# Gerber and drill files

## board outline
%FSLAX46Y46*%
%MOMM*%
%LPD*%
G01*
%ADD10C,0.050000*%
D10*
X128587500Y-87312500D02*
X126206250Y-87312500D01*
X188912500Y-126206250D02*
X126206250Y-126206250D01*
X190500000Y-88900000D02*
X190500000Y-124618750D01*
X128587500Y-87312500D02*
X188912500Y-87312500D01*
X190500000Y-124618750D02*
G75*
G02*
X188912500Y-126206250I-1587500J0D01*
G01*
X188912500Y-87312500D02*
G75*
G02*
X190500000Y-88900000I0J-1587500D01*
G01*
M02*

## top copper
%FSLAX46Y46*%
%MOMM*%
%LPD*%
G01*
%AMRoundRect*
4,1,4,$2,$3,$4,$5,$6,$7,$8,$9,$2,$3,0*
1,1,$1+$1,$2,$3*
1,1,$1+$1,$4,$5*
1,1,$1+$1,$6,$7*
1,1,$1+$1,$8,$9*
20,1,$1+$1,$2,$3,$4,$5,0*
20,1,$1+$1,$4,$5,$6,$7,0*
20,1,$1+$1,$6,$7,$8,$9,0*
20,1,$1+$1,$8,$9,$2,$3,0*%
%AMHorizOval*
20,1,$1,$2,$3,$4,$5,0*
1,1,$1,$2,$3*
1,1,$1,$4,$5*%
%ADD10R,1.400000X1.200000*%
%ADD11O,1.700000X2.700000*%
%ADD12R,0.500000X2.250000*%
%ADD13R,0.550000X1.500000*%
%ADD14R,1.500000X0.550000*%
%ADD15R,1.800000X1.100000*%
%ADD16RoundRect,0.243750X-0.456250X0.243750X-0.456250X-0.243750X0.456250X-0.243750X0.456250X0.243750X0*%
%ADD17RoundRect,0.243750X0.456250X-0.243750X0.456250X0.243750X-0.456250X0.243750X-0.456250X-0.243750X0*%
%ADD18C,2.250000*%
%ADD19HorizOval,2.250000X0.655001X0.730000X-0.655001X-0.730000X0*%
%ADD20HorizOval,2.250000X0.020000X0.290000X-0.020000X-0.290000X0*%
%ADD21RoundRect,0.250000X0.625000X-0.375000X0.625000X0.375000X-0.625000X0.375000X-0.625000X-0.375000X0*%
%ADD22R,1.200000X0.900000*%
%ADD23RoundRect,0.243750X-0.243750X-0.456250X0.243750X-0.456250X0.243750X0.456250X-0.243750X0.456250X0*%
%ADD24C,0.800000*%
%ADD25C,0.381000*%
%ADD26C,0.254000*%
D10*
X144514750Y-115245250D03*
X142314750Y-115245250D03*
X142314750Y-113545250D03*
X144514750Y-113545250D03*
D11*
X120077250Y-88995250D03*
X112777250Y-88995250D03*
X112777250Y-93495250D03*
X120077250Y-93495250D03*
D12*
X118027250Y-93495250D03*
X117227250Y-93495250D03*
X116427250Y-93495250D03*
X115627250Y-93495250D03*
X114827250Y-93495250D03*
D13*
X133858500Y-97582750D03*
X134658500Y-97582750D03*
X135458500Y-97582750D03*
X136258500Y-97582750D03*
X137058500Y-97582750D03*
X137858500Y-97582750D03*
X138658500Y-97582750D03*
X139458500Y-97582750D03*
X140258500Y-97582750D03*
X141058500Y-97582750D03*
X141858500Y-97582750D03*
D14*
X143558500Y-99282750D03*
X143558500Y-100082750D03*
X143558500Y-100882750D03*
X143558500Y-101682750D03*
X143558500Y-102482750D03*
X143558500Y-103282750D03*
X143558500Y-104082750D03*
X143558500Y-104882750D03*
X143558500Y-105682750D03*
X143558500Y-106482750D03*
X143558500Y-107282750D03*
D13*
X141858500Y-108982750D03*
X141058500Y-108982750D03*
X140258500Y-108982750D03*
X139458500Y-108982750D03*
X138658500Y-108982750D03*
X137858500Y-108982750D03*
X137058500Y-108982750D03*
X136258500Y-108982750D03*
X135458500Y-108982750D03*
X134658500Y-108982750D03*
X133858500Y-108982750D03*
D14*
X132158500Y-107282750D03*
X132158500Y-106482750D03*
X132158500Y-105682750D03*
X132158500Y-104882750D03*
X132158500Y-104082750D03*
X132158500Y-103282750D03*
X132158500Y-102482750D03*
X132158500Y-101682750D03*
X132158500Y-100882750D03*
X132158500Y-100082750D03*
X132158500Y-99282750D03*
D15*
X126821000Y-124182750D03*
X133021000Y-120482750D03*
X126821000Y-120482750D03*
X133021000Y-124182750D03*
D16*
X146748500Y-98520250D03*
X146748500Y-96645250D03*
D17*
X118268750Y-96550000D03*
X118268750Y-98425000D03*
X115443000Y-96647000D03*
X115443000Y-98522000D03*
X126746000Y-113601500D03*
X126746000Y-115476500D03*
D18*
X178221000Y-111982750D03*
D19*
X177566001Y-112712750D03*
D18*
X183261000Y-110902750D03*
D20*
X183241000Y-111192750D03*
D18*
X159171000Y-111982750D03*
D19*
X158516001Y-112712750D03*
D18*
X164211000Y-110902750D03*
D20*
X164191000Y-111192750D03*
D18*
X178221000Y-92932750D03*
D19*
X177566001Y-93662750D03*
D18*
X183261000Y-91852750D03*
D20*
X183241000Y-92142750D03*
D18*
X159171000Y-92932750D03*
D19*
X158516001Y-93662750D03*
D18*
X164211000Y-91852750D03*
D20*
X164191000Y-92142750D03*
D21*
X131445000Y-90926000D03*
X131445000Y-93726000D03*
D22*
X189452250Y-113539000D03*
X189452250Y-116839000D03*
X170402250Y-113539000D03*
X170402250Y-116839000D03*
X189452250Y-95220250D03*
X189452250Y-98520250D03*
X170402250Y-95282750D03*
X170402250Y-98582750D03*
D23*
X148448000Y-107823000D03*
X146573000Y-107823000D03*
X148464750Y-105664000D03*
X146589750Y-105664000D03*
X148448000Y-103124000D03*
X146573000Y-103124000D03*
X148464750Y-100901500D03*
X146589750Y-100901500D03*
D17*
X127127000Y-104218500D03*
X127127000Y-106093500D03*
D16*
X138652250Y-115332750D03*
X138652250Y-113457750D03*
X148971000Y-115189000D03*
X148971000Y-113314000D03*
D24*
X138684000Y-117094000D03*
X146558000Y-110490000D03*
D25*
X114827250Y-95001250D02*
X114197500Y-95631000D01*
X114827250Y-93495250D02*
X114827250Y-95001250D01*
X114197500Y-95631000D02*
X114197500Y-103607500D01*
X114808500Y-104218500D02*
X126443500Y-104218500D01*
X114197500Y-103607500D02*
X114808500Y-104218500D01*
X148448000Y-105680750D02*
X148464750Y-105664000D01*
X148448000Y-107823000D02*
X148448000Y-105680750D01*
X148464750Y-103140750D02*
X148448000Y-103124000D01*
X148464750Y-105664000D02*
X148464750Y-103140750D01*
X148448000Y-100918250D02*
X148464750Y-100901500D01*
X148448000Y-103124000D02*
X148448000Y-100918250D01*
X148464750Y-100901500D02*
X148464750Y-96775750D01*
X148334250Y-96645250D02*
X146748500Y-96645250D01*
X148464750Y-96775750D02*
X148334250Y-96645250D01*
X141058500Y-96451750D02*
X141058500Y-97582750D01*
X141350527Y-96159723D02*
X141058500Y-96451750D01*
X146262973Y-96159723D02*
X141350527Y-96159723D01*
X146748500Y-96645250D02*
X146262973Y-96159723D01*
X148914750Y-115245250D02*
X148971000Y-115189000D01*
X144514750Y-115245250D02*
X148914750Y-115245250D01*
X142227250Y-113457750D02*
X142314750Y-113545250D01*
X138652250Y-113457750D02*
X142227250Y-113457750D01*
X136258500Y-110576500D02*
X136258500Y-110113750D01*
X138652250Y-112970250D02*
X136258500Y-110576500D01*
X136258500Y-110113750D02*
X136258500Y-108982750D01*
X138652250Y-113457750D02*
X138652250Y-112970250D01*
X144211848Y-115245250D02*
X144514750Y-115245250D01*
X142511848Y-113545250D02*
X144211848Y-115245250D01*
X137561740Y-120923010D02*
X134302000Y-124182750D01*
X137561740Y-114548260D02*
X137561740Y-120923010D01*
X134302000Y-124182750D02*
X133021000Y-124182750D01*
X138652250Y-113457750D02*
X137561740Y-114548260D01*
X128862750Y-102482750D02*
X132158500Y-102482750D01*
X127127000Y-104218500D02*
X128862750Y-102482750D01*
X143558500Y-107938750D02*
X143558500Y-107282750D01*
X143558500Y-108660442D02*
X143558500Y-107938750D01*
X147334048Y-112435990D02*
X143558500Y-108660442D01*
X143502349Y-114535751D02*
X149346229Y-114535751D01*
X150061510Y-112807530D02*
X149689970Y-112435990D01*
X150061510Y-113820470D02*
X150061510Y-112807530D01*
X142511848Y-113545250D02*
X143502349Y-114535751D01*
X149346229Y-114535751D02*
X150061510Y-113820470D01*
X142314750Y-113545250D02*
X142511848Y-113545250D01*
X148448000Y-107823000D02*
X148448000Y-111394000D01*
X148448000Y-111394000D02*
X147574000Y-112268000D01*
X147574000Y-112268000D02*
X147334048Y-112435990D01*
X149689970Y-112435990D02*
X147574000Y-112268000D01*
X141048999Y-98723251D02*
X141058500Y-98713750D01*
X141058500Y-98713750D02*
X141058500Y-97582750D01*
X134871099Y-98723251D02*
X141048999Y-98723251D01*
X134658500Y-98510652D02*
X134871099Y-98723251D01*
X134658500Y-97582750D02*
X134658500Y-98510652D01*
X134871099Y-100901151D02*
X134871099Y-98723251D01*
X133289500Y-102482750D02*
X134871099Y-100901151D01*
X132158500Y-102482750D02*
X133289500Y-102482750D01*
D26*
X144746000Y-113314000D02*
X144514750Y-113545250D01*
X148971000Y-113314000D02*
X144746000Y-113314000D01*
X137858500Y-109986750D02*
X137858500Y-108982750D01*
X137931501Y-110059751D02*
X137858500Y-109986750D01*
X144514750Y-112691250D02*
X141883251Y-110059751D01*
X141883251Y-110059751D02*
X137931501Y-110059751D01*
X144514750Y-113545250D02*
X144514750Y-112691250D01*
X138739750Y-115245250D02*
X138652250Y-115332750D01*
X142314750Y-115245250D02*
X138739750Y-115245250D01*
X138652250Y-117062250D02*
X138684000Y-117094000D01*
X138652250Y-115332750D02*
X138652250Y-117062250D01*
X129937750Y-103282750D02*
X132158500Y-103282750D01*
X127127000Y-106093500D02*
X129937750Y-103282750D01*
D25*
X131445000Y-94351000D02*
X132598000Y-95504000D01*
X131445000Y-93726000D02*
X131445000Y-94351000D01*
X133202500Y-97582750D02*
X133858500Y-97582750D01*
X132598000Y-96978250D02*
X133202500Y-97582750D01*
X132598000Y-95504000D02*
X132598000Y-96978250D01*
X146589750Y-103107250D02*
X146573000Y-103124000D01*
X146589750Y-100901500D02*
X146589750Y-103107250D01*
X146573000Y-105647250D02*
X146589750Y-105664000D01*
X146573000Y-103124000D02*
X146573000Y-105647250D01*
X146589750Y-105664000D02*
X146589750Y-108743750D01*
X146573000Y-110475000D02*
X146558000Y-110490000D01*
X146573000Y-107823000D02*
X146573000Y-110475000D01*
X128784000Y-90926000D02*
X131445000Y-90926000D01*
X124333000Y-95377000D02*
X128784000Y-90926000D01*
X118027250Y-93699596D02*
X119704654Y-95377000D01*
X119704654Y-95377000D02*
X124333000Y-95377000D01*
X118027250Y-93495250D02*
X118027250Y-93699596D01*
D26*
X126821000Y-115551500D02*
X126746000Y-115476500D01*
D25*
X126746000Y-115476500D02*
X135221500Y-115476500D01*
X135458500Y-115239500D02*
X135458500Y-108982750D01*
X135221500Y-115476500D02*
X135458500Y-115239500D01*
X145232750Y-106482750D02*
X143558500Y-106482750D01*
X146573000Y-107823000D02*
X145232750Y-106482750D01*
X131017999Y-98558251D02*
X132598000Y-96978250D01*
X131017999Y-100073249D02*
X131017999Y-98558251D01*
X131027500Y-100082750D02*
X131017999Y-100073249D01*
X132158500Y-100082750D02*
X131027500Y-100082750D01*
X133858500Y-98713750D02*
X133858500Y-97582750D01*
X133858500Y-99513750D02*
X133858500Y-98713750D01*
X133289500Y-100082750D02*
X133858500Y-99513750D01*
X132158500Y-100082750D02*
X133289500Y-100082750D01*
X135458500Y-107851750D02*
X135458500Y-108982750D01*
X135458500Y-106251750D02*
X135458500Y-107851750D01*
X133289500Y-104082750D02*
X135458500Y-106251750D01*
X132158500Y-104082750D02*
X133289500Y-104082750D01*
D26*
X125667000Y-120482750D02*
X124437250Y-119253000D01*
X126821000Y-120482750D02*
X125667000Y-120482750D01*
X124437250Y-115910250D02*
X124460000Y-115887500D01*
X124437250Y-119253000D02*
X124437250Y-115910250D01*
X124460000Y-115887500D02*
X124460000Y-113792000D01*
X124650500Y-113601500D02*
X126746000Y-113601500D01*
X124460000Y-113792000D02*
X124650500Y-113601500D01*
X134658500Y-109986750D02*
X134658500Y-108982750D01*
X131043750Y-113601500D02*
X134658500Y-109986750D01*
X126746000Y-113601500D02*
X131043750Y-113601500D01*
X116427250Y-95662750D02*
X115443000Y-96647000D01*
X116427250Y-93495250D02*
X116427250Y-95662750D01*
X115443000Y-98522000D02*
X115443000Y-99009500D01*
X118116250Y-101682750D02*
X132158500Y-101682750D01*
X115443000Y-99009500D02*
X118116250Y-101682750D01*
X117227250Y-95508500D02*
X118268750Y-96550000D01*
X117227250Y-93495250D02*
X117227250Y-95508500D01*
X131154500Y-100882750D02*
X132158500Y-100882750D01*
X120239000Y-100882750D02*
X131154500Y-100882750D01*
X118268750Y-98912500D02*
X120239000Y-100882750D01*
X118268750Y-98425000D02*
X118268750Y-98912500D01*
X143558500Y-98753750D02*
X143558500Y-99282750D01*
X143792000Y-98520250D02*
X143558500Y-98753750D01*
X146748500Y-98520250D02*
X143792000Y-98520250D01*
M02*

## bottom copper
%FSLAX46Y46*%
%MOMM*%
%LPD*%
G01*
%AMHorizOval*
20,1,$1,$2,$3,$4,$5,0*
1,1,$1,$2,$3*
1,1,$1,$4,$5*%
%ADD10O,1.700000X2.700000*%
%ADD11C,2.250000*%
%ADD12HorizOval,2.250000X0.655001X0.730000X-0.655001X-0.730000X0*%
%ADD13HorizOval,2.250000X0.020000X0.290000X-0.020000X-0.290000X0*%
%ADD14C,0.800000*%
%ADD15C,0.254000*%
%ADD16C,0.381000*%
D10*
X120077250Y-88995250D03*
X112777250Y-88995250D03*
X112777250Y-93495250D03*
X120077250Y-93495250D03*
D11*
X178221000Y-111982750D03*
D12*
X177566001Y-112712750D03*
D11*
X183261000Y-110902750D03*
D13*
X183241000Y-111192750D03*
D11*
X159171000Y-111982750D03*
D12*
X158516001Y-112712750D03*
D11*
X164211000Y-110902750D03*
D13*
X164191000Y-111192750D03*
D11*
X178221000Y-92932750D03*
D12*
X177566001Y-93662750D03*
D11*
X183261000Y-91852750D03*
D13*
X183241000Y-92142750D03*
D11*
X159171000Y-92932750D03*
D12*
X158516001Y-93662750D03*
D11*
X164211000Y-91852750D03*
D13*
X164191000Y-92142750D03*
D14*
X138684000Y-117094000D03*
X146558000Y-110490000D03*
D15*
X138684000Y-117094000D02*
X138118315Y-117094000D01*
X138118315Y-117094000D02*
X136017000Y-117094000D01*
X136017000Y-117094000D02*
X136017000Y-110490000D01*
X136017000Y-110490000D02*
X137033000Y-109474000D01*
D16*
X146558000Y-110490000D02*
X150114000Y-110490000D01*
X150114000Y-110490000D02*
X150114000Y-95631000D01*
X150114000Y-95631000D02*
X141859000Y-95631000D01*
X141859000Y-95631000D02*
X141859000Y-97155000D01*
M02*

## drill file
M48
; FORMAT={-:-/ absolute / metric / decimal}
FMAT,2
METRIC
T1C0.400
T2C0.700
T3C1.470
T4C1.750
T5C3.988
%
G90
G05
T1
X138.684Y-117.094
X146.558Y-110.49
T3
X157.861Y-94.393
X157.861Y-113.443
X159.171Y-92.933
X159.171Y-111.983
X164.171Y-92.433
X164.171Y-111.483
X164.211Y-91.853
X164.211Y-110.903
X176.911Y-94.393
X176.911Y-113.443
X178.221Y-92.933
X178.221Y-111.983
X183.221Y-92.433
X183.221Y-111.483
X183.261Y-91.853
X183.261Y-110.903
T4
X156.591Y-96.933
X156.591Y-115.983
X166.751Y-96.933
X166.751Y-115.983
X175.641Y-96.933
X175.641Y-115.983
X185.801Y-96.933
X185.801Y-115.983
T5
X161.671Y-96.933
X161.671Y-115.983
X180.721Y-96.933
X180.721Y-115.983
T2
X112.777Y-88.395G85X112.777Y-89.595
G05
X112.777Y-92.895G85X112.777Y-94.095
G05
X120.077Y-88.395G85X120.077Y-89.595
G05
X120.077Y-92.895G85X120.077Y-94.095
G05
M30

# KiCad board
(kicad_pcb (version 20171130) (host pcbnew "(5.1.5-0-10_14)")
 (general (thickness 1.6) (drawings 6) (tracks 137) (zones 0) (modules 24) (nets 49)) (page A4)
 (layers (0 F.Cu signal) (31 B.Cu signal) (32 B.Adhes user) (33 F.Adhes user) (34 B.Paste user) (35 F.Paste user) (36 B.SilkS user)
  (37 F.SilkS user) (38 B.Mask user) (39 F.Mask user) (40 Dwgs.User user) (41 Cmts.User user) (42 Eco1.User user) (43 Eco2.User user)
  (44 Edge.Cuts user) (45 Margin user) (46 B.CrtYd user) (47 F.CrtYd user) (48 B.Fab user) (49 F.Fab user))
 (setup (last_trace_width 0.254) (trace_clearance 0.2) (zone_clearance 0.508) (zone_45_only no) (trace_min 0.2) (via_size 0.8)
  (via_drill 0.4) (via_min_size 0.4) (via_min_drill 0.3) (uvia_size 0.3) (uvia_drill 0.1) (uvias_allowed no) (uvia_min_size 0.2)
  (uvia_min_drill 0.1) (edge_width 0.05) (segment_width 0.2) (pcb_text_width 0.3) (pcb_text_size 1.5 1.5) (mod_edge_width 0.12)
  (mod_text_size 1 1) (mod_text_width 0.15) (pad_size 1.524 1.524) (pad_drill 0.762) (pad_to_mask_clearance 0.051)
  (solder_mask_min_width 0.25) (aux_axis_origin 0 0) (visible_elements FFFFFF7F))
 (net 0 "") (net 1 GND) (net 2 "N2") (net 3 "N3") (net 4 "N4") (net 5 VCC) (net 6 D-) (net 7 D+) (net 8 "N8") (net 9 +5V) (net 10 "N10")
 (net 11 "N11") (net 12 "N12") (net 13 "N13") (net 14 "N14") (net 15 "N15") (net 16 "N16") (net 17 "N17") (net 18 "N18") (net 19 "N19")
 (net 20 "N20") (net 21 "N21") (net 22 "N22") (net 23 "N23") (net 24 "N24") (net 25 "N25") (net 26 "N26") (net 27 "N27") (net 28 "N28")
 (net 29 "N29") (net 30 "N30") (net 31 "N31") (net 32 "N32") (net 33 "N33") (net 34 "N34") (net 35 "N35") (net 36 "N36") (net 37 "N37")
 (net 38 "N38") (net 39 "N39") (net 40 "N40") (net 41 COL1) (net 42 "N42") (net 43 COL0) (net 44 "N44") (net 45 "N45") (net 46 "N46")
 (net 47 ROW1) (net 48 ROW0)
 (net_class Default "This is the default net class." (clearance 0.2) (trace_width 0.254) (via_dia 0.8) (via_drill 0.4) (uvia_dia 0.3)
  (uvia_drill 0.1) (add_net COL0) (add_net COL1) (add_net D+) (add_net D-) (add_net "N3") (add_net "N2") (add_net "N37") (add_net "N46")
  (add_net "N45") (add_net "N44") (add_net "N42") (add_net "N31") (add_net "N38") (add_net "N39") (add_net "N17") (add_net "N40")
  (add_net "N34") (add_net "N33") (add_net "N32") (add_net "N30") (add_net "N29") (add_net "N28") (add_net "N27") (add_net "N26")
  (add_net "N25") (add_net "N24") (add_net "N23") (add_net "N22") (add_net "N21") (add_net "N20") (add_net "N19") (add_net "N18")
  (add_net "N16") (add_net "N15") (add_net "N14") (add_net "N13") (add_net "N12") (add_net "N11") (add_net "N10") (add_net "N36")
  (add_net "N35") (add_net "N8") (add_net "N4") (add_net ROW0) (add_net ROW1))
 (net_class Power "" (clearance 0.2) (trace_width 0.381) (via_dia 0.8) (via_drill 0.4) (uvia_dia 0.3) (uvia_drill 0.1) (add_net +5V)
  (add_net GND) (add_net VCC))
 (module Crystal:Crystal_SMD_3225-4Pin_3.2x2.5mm (layer F.Cu) (at 143.41475 114.39525 180)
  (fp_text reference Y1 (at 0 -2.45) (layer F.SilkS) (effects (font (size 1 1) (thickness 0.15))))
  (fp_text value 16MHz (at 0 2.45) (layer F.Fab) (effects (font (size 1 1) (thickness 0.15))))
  (pad 4 smd rect (at -1.1 -0.85 180) (size 1.4 1.2) (layers F.Cu F.Paste F.Mask) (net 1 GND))
  (pad 3 smd rect (at 1.1 -0.85 180) (size 1.4 1.2) (layers F.Cu F.Paste F.Mask) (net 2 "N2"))
  (pad 2 smd rect (at 1.1 0.85 180) (size 1.4 1.2) (layers F.Cu F.Paste F.Mask) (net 1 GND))
  (pad 1 smd rect (at -1.1 0.85 180) (size 1.4 1.2) (layers F.Cu F.Paste F.Mask) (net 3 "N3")))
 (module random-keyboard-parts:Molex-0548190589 (layer F.Cu) (at 116.42725 88.99525 270)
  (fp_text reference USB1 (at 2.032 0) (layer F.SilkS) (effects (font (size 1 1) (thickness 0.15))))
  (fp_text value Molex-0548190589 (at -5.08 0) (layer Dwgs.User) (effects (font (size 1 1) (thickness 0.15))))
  (pad 6 thru_hole oval (at 0 -3.65 270) (size 2.7 1.7) (drill oval 1.9 0.7) (layers *.Cu *.Mask) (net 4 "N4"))
  (pad 6 thru_hole oval (at 0 3.65 270) (size 2.7 1.7) (drill oval 1.9 0.7) (layers *.Cu *.Mask) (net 4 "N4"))
  (pad 6 thru_hole oval (at 4.5 3.65 270) (size 2.7 1.7) (drill oval 1.9 0.7) (layers *.Cu *.Mask) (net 4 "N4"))
  (pad 6 thru_hole oval (at 4.5 -3.65 270) (size 2.7 1.7) (drill oval 1.9 0.7) (layers *.Cu *.Mask) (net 4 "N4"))
  (pad 5 smd rect (at 4.5 -1.6 270) (size 2.25 0.5) (layers F.Cu F.Paste F.Mask) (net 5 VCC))
  (pad 4 smd rect (at 4.5 -0.8 270) (size 2.25 0.5) (layers F.Cu F.Paste F.Mask) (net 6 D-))
  (pad 3 smd rect (at 4.5 0 270) (size 2.25 0.5) (layers F.Cu F.Paste F.Mask) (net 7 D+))
  (pad 2 smd rect (at 4.5 0.8 270) (size 2.25 0.5) (layers F.Cu F.Paste F.Mask) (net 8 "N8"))
  (pad 1 smd rect (at 4.5 1.6 270) (size 2.25 0.5) (layers F.Cu F.Paste F.Mask) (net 1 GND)))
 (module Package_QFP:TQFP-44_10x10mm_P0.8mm (layer F.Cu) (at 137.8585 103.28275)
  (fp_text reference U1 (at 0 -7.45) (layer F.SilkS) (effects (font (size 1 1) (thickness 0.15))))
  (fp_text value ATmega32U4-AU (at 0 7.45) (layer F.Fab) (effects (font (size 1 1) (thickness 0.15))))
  (pad 44 smd rect (at -4 -5.7 90) (size 1.5 0.55) (layers F.Cu F.Paste F.Mask) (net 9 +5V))
  (pad 43 smd rect (at -3.2 -5.7 90) (size 1.5 0.55) (layers F.Cu F.Paste F.Mask) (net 1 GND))
  (pad 42 smd rect (at -2.4 -5.7 90) (size 1.5 0.55) (layers F.Cu F.Paste F.Mask) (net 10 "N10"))
  (pad 41 smd rect (at -1.6 -5.7 90) (size 1.5 0.55) (layers F.Cu F.Paste F.Mask) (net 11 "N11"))
  (pad 40 smd rect (at -0.8 -5.7 90) (size 1.5 0.55) (layers F.Cu F.Paste F.Mask) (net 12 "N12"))
  (pad 39 smd rect (at 0 -5.7 90) (size 1.5 0.55) (layers F.Cu F.Paste F.Mask) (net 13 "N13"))
  (pad 38 smd rect (at 0.8 -5.7 90) (size 1.5 0.55) (layers F.Cu F.Paste F.Mask) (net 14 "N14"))
  (pad 37 smd rect (at 1.6 -5.7 90) (size 1.5 0.55) (layers F.Cu F.Paste F.Mask) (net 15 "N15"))
  (pad 36 smd rect (at 2.4 -5.7 90) (size 1.5 0.55) (layers F.Cu F.Paste F.Mask) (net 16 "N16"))
  (pad 35 smd rect (at 3.2 -5.7 90) (size 1.5 0.55) (layers F.Cu F.Paste F.Mask) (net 1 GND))
  (pad 34 smd rect (at 4 -5.7 90) (size 1.5 0.55) (layers F.Cu F.Paste F.Mask) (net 9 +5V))
  (pad 33 smd rect (at 5.7 -4) (size 1.5 0.55) (layers F.Cu F.Paste F.Mask) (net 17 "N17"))
  (pad 32 smd rect (at 5.7 -3.2) (size 1.5 0.55) (layers F.Cu F.Paste F.Mask) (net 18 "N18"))
  (pad 31 smd rect (at 5.7 -2.4) (size 1.5 0.55) (layers F.Cu F.Paste F.Mask) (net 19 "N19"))
  (pad 30 smd rect (at 5.7 -1.6) (size 1.5 0.55) (layers F.Cu F.Paste F.Mask) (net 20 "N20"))
  (pad 29 smd rect (at 5.7 -0.8) (size 1.5 0.55) (layers F.Cu F.Paste F.Mask) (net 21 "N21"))
  (pad 28 smd rect (at 5.7 0) (size 1.5 0.55) (layers F.Cu F.Paste F.Mask) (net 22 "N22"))
  (pad 27 smd rect (at 5.7 0.8) (size 1.5 0.55) (layers F.Cu F.Paste F.Mask) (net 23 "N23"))
  (pad 26 smd rect (at 5.7 1.6) (size 1.5 0.55) (layers F.Cu F.Paste F.Mask) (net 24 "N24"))
  (pad 25 smd rect (at 5.7 2.4) (size 1.5 0.55) (layers F.Cu F.Paste F.Mask) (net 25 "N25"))
  (pad 24 smd rect (at 5.7 3.2) (size 1.5 0.55) (layers F.Cu F.Paste F.Mask) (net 9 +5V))
  (pad 23 smd rect (at 5.7 4) (size 1.5 0.55) (layers F.Cu F.Paste F.Mask) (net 1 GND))
  (pad 22 smd rect (at 4 5.7 90) (size 1.5 0.55) (layers F.Cu F.Paste F.Mask) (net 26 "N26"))
  (pad 21 smd rect (at 3.2 5.7 90) (size 1.5 0.55) (layers F.Cu F.Paste F.Mask) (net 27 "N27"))
  (pad 20 smd rect (at 2.4 5.7 90) (size 1.5 0.55) (layers F.Cu F.Paste F.Mask) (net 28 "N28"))
  (pad 19 smd rect (at 1.6 5.7 90) (size 1.5 0.55) (layers F.Cu F.Paste F.Mask) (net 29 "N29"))
  (pad 18 smd rect (at 0.8 5.7 90) (size 1.5 0.55) (layers F.Cu F.Paste F.Mask) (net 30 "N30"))
  (pad 17 smd rect (at 0 5.7 90) (size 1.5 0.55) (layers F.Cu F.Paste F.Mask) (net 3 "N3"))
  (pad 16 smd rect (at -0.8 5.7 90) (size 1.5 0.55) (layers F.Cu F.Paste F.Mask) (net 2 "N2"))
  (pad 15 smd rect (at -1.6 5.7 90) (size 1.5 0.55) (layers F.Cu F.Paste F.Mask) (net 1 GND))
  (pad 14 smd rect (at -2.4 5.7 90) (size 1.5 0.55) (layers F.Cu F.Paste F.Mask) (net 9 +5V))
  (pad 13 smd rect (at -3.2 5.7 90) (size 1.5 0.55) (layers F.Cu F.Paste F.Mask) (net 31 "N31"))
  (pad 12 smd rect (at -4 5.7 90) (size 1.5 0.55) (layers F.Cu F.Paste F.Mask) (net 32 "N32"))
  (pad 11 smd rect (at -5.7 4) (size 1.5 0.55) (layers F.Cu F.Paste F.Mask) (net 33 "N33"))
  (pad 10 smd rect (at -5.7 3.2) (size 1.5 0.55) (layers F.Cu F.Paste F.Mask) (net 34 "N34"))
  (pad 9 smd rect (at -5.7 2.4) (size 1.5 0.55) (layers F.Cu F.Paste F.Mask) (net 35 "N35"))
  (pad 8 smd rect (at -5.7 1.6) (size 1.5 0.55) (layers F.Cu F.Paste F.Mask) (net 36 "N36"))
  (pad 7 smd rect (at -5.7 0.8) (size 1.5 0.55) (layers F.Cu F.Paste F.Mask) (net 9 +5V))
  (pad 6 smd rect (at -5.7 0) (size 1.5 0.55) (layers F.Cu F.Paste F.Mask) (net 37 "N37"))
  (pad 5 smd rect (at -5.7 -0.8) (size 1.5 0.55) (layers F.Cu F.Paste F.Mask) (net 1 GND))
  (pad 4 smd rect (at -5.7 -1.6) (size 1.5 0.55) (layers F.Cu F.Paste F.Mask) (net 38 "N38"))
  (pad 3 smd rect (at -5.7 -2.4) (size 1.5 0.55) (layers F.Cu F.Paste F.Mask) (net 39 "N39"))
  (pad 2 smd rect (at -5.7 -3.2) (size 1.5 0.55) (layers F.Cu F.Paste F.Mask) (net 9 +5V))
  (pad 1 smd rect (at -5.7 -4) (size 1.5 0.55) (layers F.Cu F.Paste F.Mask) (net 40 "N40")))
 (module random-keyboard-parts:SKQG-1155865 (layer F.Cu) (at 129.921 122.33275)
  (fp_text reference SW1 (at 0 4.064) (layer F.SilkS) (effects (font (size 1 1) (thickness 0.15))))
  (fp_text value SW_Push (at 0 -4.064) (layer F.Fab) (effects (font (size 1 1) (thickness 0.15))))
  (pad 4 smd rect (at -3.1 1.85) (size 1.8 1.1) (layers F.Cu F.Paste F.Mask))
  (pad 3 smd rect (at 3.1 -1.85) (size 1.8 1.1) (layers F.Cu F.Paste F.Mask))
  (pad 2 smd rect (at -3.1 -1.85) (size 1.8 1.1) (layers F.Cu F.Paste F.Mask) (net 31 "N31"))
  (pad 1 smd rect (at 3.1 1.85) (size 1.8 1.1) (layers F.Cu F.Paste F.Mask) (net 1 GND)))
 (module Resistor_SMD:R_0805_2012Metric (layer F.Cu) (at 146.7485 97.58275 270)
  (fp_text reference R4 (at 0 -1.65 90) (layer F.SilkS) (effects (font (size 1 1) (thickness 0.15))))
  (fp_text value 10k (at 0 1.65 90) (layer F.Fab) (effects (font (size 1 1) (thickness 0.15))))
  (pad 2 smd roundrect (at 0.9375 0 270) (size 0.975 1.4) (layers F.Cu F.Paste F.Mask) (roundrect_rratio 0.25) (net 17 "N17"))
  (pad 1 smd roundrect (at -0.9375 0 270) (size 0.975 1.4) (layers F.Cu F.Paste F.Mask) (roundrect_rratio 0.25) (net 1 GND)))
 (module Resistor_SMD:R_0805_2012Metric (layer F.Cu) (at 118.26875 97.4875 90)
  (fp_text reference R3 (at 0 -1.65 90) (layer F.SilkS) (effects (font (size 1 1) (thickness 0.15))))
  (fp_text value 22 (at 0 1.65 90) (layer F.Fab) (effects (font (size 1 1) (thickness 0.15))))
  (pad 2 smd roundrect (at 0.9375 0 90) (size 0.975 1.4) (layers F.Cu F.Paste F.Mask) (roundrect_rratio 0.25) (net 6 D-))
  (pad 1 smd roundrect (at -0.9375 0 90) (size 0.975 1.4) (layers F.Cu F.Paste F.Mask) (roundrect_rratio 0.25) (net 39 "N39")))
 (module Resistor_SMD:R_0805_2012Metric (layer F.Cu) (at 115.443 97.5845 90)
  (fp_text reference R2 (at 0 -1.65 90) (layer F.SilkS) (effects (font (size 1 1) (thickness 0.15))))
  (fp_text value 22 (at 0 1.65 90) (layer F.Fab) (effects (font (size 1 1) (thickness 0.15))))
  (pad 2 smd roundrect (at 0.9375 0 90) (size 0.975 1.4) (layers F.Cu F.Paste F.Mask) (roundrect_rratio 0.25) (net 7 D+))
  (pad 1 smd roundrect (at -0.9375 0 90) (size 0.975 1.4) (layers F.Cu F.Paste F.Mask) (roundrect_rratio 0.25) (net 38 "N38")))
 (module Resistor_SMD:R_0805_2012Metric (layer F.Cu) (at 126.746 114.539 90)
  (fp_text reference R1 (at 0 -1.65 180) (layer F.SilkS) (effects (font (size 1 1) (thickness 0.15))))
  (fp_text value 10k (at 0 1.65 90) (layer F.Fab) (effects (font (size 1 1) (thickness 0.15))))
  (pad 2 smd roundrect (at 0.9375 0 90) (size 0.975 1.4) (layers F.Cu F.Paste F.Mask) (roundrect_rratio 0.25) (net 31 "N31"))
  (pad 1 smd roundrect (at -0.9375 0 90) (size 0.975 1.4) (layers F.Cu F.Paste F.Mask) (roundrect_rratio 0.25) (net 9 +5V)))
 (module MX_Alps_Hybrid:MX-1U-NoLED (layer F.Cu) (at 180.721 115.98275)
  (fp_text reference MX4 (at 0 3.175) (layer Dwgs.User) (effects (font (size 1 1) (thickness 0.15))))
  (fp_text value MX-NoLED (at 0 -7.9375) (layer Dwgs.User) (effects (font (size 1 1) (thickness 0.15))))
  (pad "" np_thru_hole circle (at 5.08 0 48.0996) (size 1.75 1.75) (drill 1.75) (layers *.Cu *.Mask))
  (pad "" np_thru_hole circle (at -5.08 0 48.0996) (size 1.75 1.75) (drill 1.75) (layers *.Cu *.Mask))
  (pad 1 thru_hole circle (at -2.5 -4) (size 2.25 2.25) (drill 1.47) (layers *.Cu B.Mask) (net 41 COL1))
  (pad "" np_thru_hole circle (at 0 0) (size 3.9878 3.9878) (drill 3.9878) (layers *.Cu *.Mask))
  (pad 1 thru_hole oval (at -3.81 -2.54 48.0996) (size 4.211556 2.25) (drill 1.47 (offset 0.980778 0)) (layers *.Cu B.Mask) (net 41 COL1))
  (pad 2 thru_hole circle (at 2.54 -5.08) (size 2.25 2.25) (drill 1.47) (layers *.Cu B.Mask) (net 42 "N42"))
  (pad 2 thru_hole oval (at 2.5 -4.5 86.0548) (size 2.831378 2.25) (drill 1.47 (offset 0.290689 0)) (layers *.Cu B.Mask) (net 42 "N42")))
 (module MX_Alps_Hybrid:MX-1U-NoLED (layer F.Cu) (at 161.671 115.98275)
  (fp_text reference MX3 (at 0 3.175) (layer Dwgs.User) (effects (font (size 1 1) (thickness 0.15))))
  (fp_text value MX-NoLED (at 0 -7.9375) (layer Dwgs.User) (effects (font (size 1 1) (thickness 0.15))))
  (pad "" np_thru_hole circle (at 5.08 0 48.0996) (size 1.75 1.75) (drill 1.75) (layers *.Cu *.Mask))
  (pad "" np_thru_hole circle (at -5.08 0 48.0996) (size 1.75 1.75) (drill 1.75) (layers *.Cu *.Mask))
  (pad 1 thru_hole circle (at -2.5 -4) (size 2.25 2.25) (drill 1.47) (layers *.Cu B.Mask) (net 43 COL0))
  (pad "" np_thru_hole circle (at 0 0) (size 3.9878 3.9878) (drill 3.9878) (layers *.Cu *.Mask))
  (pad 1 thru_hole oval (at -3.81 -2.54 48.0996) (size 4.211556 2.25) (drill 1.47 (offset 0.980778 0)) (layers *.Cu B.Mask) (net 43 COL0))
  (pad 2 thru_hole circle (at 2.54 -5.08) (size 2.25 2.25) (drill 1.47) (layers *.Cu B.Mask) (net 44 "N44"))
  (pad 2 thru_hole oval (at 2.5 -4.5 86.0548) (size 2.831378 2.25) (drill 1.47 (offset 0.290689 0)) (layers *.Cu B.Mask) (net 44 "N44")))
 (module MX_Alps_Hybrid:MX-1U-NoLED (layer F.Cu) (at 180.721 96.93275)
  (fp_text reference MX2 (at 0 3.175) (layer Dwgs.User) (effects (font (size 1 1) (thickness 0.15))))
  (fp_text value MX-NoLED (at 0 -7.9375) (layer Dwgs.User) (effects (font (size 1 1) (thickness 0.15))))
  (pad "" np_thru_hole circle (at 5.08 0 48.0996) (size 1.75 1.75) (drill 1.75) (layers *.Cu *.Mask))
  (pad "" np_thru_hole circle (at -5.08 0 48.0996) (size 1.75 1.75) (drill 1.75) (layers *.Cu *.Mask))
  (pad 1 thru_hole circle (at -2.5 -4) (size 2.25 2.25) (drill 1.47) (layers *.Cu B.Mask) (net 41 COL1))
  (pad "" np_thru_hole circle (at 0 0) (size 3.9878 3.9878) (drill 3.9878) (layers *.Cu *.Mask))
  (pad 1 thru_hole oval (at -3.81 -2.54 48.0996) (size 4.211556 2.25) (drill 1.47 (offset 0.980778 0)) (layers *.Cu B.Mask) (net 41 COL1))
  (pad 2 thru_hole circle (at 2.54 -5.08) (size 2.25 2.25) (drill 1.47) (layers *.Cu B.Mask) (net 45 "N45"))
  (pad 2 thru_hole oval (at 2.5 -4.5 86.0548) (size 2.831378 2.25) (drill 1.47 (offset 0.290689 0)) (layers *.Cu B.Mask) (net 45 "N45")))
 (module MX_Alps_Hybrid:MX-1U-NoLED (layer F.Cu) (at 161.671 96.93275)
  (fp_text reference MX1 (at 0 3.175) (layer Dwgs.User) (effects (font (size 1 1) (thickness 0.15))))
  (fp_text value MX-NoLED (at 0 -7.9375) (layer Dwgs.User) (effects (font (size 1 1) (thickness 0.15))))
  (pad "" np_thru_hole circle (at 5.08 0 48.0996) (size 1.75 1.75) (drill 1.75) (layers *.Cu *.Mask))
  (pad "" np_thru_hole circle (at -5.08 0 48.0996) (size 1.75 1.75) (drill 1.75) (layers *.Cu *.Mask))
  (pad 1 thru_hole circle (at -2.5 -4) (size 2.25 2.25) (drill 1.47) (layers *.Cu B.Mask) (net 43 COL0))
  (pad "" np_thru_hole circle (at 0 0) (size 3.9878 3.9878) (drill 3.9878) (layers *.Cu *.Mask))
  (pad 1 thru_hole oval (at -3.81 -2.54 48.0996) (size 4.211556 2.25) (drill 1.47 (offset 0.980778 0)) (layers *.Cu B.Mask) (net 43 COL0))
  (pad 2 thru_hole circle (at 2.54 -5.08) (size 2.25 2.25) (drill 1.47) (layers *.Cu B.Mask) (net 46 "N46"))
  (pad 2 thru_hole oval (at 2.5 -4.5 86.0548) (size 2.831378 2.25) (drill 1.47 (offset 0.290689 0)) (layers *.Cu B.Mask) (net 46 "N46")))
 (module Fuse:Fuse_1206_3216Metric (layer F.Cu) (at 131.445 92.326 90)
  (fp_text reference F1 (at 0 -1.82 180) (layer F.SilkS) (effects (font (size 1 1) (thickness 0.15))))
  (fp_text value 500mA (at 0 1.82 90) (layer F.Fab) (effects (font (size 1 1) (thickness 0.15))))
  (pad 2 smd roundrect (at 1.4 0 90) (size 1.25 1.75) (layers F.Cu F.Paste F.Mask) (roundrect_rratio 0.2) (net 5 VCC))
  (pad 1 smd roundrect (at -1.4 0 90) (size 1.25 1.75) (layers F.Cu F.Paste F.Mask) (roundrect_rratio 0.2) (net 9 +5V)))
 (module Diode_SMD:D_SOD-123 (layer F.Cu) (at 189.45225 115.189 90)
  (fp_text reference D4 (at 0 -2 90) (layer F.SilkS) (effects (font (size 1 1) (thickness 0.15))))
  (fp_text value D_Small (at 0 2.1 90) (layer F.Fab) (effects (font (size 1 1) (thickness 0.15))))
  (pad 2 smd rect (at 1.65 0 90) (size 0.9 1.2) (layers F.Cu F.Paste F.Mask) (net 42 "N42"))
  (pad 1 smd rect (at -1.65 0 90) (size 0.9 1.2) (layers F.Cu F.Paste F.Mask) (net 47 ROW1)))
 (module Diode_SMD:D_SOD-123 (layer F.Cu) (at 170.40225 115.189 90)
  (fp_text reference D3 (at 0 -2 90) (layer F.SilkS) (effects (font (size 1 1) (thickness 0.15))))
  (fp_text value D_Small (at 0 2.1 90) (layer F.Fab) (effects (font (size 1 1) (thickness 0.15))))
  (pad 2 smd rect (at 1.65 0 90) (size 0.9 1.2) (layers F.Cu F.Paste F.Mask) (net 44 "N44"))
  (pad 1 smd rect (at -1.65 0 90) (size 0.9 1.2) (layers F.Cu F.Paste F.Mask) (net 47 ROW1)))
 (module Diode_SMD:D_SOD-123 (layer F.Cu) (at 189.45225 96.87025 90)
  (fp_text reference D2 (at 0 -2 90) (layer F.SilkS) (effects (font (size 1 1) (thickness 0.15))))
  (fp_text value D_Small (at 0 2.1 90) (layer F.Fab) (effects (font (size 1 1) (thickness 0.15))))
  (pad 2 smd rect (at 1.65 0 90) (size 0.9 1.2) (layers F.Cu F.Paste F.Mask) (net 45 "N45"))
  (pad 1 smd rect (at -1.65 0 90) (size 0.9 1.2) (layers F.Cu F.Paste F.Mask) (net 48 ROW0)))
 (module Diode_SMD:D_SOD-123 (layer F.Cu) (at 170.40225 96.93275 90)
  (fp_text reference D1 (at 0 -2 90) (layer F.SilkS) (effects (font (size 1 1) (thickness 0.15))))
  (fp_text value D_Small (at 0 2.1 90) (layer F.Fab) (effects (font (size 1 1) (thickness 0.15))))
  (pad 2 smd rect (at 1.65 0 90) (size 0.9 1.2) (layers F.Cu F.Paste F.Mask) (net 46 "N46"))
  (pad 1 smd rect (at -1.65 0 90) (size 0.9 1.2) (layers F.Cu F.Paste F.Mask) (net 48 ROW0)))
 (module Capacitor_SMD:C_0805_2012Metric (layer F.Cu) (at 147.5105 107.823)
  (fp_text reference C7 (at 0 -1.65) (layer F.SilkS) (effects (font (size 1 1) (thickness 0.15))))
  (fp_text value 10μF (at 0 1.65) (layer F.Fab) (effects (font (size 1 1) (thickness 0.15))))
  (pad 2 smd roundrect (at 0.9375 0) (size 0.975 1.4) (layers F.Cu F.Paste F.Mask) (roundrect_rratio 0.25) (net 1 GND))
  (pad 1 smd roundrect (at -0.9375 0) (size 0.975 1.4) (layers F.Cu F.Paste F.Mask) (roundrect_rratio 0.25) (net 9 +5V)))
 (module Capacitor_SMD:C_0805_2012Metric (layer F.Cu) (at 147.52725 105.664)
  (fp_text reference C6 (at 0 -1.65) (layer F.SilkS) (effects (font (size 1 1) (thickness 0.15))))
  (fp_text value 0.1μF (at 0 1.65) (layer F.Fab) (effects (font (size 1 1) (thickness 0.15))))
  (pad 2 smd roundrect (at 0.9375 0) (size 0.975 1.4) (layers F.Cu F.Paste F.Mask) (roundrect_rratio 0.25) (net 1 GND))
  (pad 1 smd roundrect (at -0.9375 0) (size 0.975 1.4) (layers F.Cu F.Paste F.Mask) (roundrect_rratio 0.25) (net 9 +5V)))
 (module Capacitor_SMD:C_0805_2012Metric (layer F.Cu) (at 147.5105 103.124)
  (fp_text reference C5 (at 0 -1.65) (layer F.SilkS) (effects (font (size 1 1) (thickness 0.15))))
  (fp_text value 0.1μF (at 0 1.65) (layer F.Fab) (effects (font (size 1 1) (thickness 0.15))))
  (pad 2 smd roundrect (at 0.9375 0) (size 0.975 1.4) (layers F.Cu F.Paste F.Mask) (roundrect_rratio 0.25) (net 1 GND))
  (pad 1 smd roundrect (at -0.9375 0) (size 0.975 1.4) (layers F.Cu F.Paste F.Mask) (roundrect_rratio 0.25) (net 9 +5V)))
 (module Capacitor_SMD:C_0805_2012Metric (layer F.Cu) (at 147.52725 100.9015)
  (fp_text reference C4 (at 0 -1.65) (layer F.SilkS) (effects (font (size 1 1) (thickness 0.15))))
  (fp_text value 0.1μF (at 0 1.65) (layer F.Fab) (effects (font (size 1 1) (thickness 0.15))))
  (pad 2 smd roundrect (at 0.9375 0) (size 0.975 1.4) (layers F.Cu F.Paste F.Mask) (roundrect_rratio 0.25) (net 1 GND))
  (pad 1 smd roundrect (at -0.9375 0) (size 0.975 1.4) (layers F.Cu F.Paste F.Mask) (roundrect_rratio 0.25) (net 9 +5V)))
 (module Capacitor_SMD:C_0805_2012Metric (layer F.Cu) (at 127.127 105.156 90)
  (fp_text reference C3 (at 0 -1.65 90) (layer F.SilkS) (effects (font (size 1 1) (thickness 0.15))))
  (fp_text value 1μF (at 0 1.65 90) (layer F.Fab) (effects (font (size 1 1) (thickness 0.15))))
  (pad 2 smd roundrect (at 0.9375 0 90) (size 0.975 1.4) (layers F.Cu F.Paste F.Mask) (roundrect_rratio 0.25) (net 1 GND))
  (pad 1 smd roundrect (at -0.9375 0 90) (size 0.975 1.4) (layers F.Cu F.Paste F.Mask) (roundrect_rratio 0.25) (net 37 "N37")))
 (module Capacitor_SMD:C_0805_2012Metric (layer F.Cu) (at 138.65225 114.39525 270)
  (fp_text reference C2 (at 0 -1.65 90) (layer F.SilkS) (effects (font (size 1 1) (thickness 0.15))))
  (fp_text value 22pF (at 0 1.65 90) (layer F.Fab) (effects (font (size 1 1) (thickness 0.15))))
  (pad 2 smd roundrect (at 0.9375 0 270) (size 0.975 1.4) (layers F.Cu F.Paste F.Mask) (roundrect_rratio 0.25) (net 2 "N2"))
  (pad 1 smd roundrect (at -0.9375 0 270) (size 0.975 1.4) (layers F.Cu F.Paste F.Mask) (roundrect_rratio 0.25) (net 1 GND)))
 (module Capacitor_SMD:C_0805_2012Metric (layer F.Cu) (at 148.971 114.2515 270)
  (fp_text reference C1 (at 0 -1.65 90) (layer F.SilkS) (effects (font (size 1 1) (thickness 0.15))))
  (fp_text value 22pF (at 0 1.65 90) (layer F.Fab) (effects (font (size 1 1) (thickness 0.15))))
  (pad 2 smd roundrect (at 0.9375 0 270) (size 0.975 1.4) (layers F.Cu F.Paste F.Mask) (roundrect_rratio 0.25) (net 1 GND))
  (pad 1 smd roundrect (at -0.9375 0 270) (size 0.975 1.4) (layers F.Cu F.Paste F.Mask) (roundrect_rratio 0.25) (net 3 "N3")))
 (gr_line (start 128.5875 87.3125) (end 126.20625 87.3125) (layer Edge.Cuts) (width 0.05))
 (gr_line (start 188.9125 126.20625) (end 126.20625 126.20625) (layer Edge.Cuts) (width 0.05))
 (gr_line (start 190.5 88.9) (end 190.5 124.61875) (layer Edge.Cuts) (width 0.05))
 (gr_line (start 128.5875 87.3125) (end 188.9125 87.3125) (layer Edge.Cuts) (width 0.05))
 (gr_arc (start 188.9125 124.61875) (end 188.9125 126.20625) (angle -90) (layer Edge.Cuts) (width 0.05))
 (gr_arc (start 188.9125 88.9) (end 190.5 88.9) (angle -90) (layer Edge.Cuts) (width 0.05))
 (segment (start 114.82725 95.00125) (end 114.1975 95.631) (width 0.381) (layer F.Cu) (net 1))
 (segment (start 114.82725 93.49525) (end 114.82725 95.00125) (width 0.381) (layer F.Cu) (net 1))
 (segment (start 114.1975 95.631) (end 114.1975 103.6075) (width 0.381) (layer F.Cu) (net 1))
 (segment (start 114.8085 104.2185) (end 126.4435 104.2185) (width 0.381) (layer F.Cu) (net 1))
 (segment (start 114.1975 103.6075) (end 114.8085 104.2185) (width 0.381) (layer F.Cu) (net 1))
 (segment (start 148.448 105.68075) (end 148.46475 105.664) (width 0.381) (layer F.Cu) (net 1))
 (segment (start 148.448 107.823) (end 148.448 105.68075) (width 0.381) (layer F.Cu) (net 1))
 (segment (start 148.46475 103.14075) (end 148.448 103.124) (width 0.381) (layer F.Cu) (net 1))
 (segment (start 148.46475 105.664) (end 148.46475 103.14075) (width 0.381) (layer F.Cu) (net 1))
 (segment (start 148.448 100.91825) (end 148.46475 100.9015) (width 0.381) (layer F.Cu) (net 1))
 (segment (start 148.448 103.124) (end 148.448 100.91825) (width 0.381) (layer F.Cu) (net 1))
 (segment (start 148.46475 100.9015) (end 148.46475 96.77575) (width 0.381) (layer F.Cu) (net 1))
 (segment (start 148.33425 96.64525) (end 146.7485 96.64525) (width 0.381) (layer F.Cu) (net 1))
 (segment (start 148.46475 96.77575) (end 148.33425 96.64525) (width 0.381) (layer F.Cu) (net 1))
 (segment (start 141.0585 96.45175) (end 141.0585 97.58275) (width 0.381) (layer F.Cu) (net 1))
 (segment (start 141.350527 96.159723) (end 141.0585 96.45175) (width 0.381) (layer F.Cu) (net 1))
 (segment (start 146.262973 96.159723) (end 141.350527 96.159723) (width 0.381) (layer F.Cu) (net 1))
 (segment (start 146.7485 96.64525) (end 146.262973 96.159723) (width 0.381) (layer F.Cu) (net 1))
 (segment (start 148.91475 115.24525) (end 148.971 115.189) (width 0.381) (layer F.Cu) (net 1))
 (segment (start 144.51475 115.24525) (end 148.91475 115.24525) (width 0.381) (layer F.Cu) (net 1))
 (segment (start 142.22725 113.45775) (end 142.31475 113.54525) (width 0.381) (layer F.Cu) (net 1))
 (segment (start 138.65225 113.45775) (end 142.22725 113.45775) (width 0.381) (layer F.Cu) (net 1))
 (segment (start 136.2585 110.5765) (end 136.2585 110.11375) (width 0.381) (layer F.Cu) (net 1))
 (segment (start 138.65225 112.97025) (end 136.2585 110.5765) (width 0.381) (layer F.Cu) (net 1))
 (segment (start 136.2585 110.11375) (end 136.2585 108.98275) (width 0.381) (layer F.Cu) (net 1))
 (segment (start 138.65225 113.45775) (end 138.65225 112.97025) (width 0.381) (layer F.Cu) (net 1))
 (segment (start 144.211848 115.24525) (end 144.51475 115.24525) (width 0.381) (layer F.Cu) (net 1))
 (segment (start 142.511848 113.54525) (end 144.211848 115.24525) (width 0.381) (layer F.Cu) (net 1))
 (segment (start 137.56174 120.92301) (end 134.302 124.18275) (width 0.381) (layer F.Cu) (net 1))
 (segment (start 137.56174 114.54826) (end 137.56174 120.92301) (width 0.381) (layer F.Cu) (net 1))
 (segment (start 134.302 124.18275) (end 133.021 124.18275) (width 0.381) (layer F.Cu) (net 1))
 (segment (start 138.65225 113.45775) (end 137.56174 114.54826) (width 0.381) (layer F.Cu) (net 1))
 (segment (start 128.86275 102.48275) (end 132.1585 102.48275) (width 0.381) (layer F.Cu) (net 1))
 (segment (start 127.127 104.2185) (end 128.86275 102.48275) (width 0.381) (layer F.Cu) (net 1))
 (segment (start 143.5585 107.93875) (end 143.5585 107.28275) (width 0.381) (layer F.Cu) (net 1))
 (segment (start 143.5585 108.660442) (end 143.5585 107.93875) (width 0.381) (layer F.Cu) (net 1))
 (segment (start 147.334048 112.43599) (end 143.5585 108.660442) (width 0.381) (layer F.Cu) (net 1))
 (segment (start 143.502349 114.535751) (end 149.346229 114.535751) (width 0.381) (layer F.Cu) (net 1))
 (segment (start 150.06151 112.80753) (end 149.68997 112.43599) (width 0.381) (layer F.Cu) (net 1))
 (segment (start 150.06151 113.82047) (end 150.06151 112.80753) (width 0.381) (layer F.Cu) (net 1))
 (segment (start 142.511848 113.54525) (end 143.502349 114.535751) (width 0.381) (layer F.Cu) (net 1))
 (segment (start 149.346229 114.535751) (end 150.06151 113.82047) (width 0.381) (layer F.Cu) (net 1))
 (segment (start 142.31475 113.54525) (end 142.511848 113.54525) (width 0.381) (layer F.Cu) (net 1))
 (segment (start 148.448 107.823) (end 148.448 111.394) (width 0.381) (layer F.Cu) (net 1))
 (segment (start 148.448 111.394) (end 147.574 112.268) (width 0.381) (layer F.Cu) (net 1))
 (segment (start 147.574 112.268) (end 147.334048 112.43599) (width 0.381) (layer F.Cu) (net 1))
 (segment (start 149.68997 112.43599) (end 147.574 112.268) (width 0.381) (layer F.Cu) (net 1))
 (segment (start 141.048999 98.723251) (end 141.0585 98.71375) (width 0.381) (layer F.Cu) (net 1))
 (segment (start 141.0585 98.71375) (end 141.0585 97.58275) (width 0.381) (layer F.Cu) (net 1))
 (segment (start 134.871099 98.723251) (end 141.048999 98.723251) (width 0.381) (layer F.Cu) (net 1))
 (segment (start 134.6585 98.510652) (end 134.871099 98.723251) (width 0.381) (layer F.Cu) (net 1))
 (segment (start 134.6585 97.58275) (end 134.6585 98.510652) (width 0.381) (layer F.Cu) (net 1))
 (segment (start 134.871099 100.901151) (end 134.871099 98.723251) (width 0.381) (layer F.Cu) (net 1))
 (segment (start 133.2895 102.48275) (end 134.871099 100.901151) (width 0.381) (layer F.Cu) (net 1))
 (segment (start 132.1585 102.48275) (end 133.2895 102.48275) (width 0.381) (layer F.Cu) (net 1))
 (segment (start 144.746 113.314) (end 144.51475 113.54525) (width 0.254) (layer F.Cu) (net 3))
 (segment (start 148.971 113.314) (end 144.746 113.314) (width 0.254) (layer F.Cu) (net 3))
 (segment (start 137.8585 109.98675) (end 137.8585 108.98275) (width 0.254) (layer F.Cu) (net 3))
 (segment (start 137.931501 110.059751) (end 137.8585 109.98675) (width 0.254) (layer F.Cu) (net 3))
 (segment (start 144.51475 112.69125) (end 141.883251 110.059751) (width 0.254) (layer F.Cu) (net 3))
 (segment (start 141.883251 110.059751) (end 137.931501 110.059751) (width 0.254) (layer F.Cu) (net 3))
 (segment (start 144.51475 113.54525) (end 144.51475 112.69125) (width 0.254) (layer F.Cu) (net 3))
 (segment (start 138.73975 115.24525) (end 138.65225 115.33275) (width 0.254) (layer F.Cu) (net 2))
 (segment (start 142.31475 115.24525) (end 138.73975 115.24525) (width 0.254) (layer F.Cu) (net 2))
 (via (at 138.684 117.094) (size 0.8) (drill 0.4) (layers F.Cu B.Cu) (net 2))
 (segment (start 138.65225 117.06225) (end 138.684 117.094) (width 0.254) (layer F.Cu) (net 2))
 (segment (start 138.65225 115.33275) (end 138.65225 117.06225) (width 0.254) (layer F.Cu) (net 2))
 (segment (start 138.684 117.094) (end 138.118315 117.094) (width 0.254) (layer B.Cu) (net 2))
 (segment (start 138.118315 117.094) (end 136.017 117.094) (width 0.254) (layer B.Cu) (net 2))
 (segment (start 136.017 117.094) (end 136.017 110.49) (width 0.254) (layer B.Cu) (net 2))
 (segment (start 136.017 110.49) (end 137.033 109.474) (width 0.254) (layer B.Cu) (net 2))
 (segment (start 129.93775 103.28275) (end 132.1585 103.28275) (width 0.254) (layer F.Cu) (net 37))
 (segment (start 127.127 106.0935) (end 129.93775 103.28275) (width 0.254) (layer F.Cu) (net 37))
 (segment (start 131.445 94.351) (end 132.598 95.504) (width 0.381) (layer F.Cu) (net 9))
 (segment (start 131.445 93.726) (end 131.445 94.351) (width 0.381) (layer F.Cu) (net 9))
 (segment (start 133.2025 97.58275) (end 133.8585 97.58275) (width 0.381) (layer F.Cu) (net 9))
 (segment (start 132.598 96.97825) (end 133.2025 97.58275) (width 0.381) (layer F.Cu) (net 9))
 (segment (start 132.598 95.504) (end 132.598 96.97825) (width 0.381) (layer F.Cu) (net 9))
 (segment (start 146.58975 103.10725) (end 146.573 103.124) (width 0.381) (layer F.Cu) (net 9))
 (segment (start 146.58975 100.9015) (end 146.58975 103.10725) (width 0.381) (layer F.Cu) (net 9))
 (segment (start 146.573 105.64725) (end 146.58975 105.664) (width 0.381) (layer F.Cu) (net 9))
 (segment (start 146.573 103.124) (end 146.573 105.64725) (width 0.381) (layer F.Cu) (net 9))
 (segment (start 146.58975 105.664) (end 146.58975 108.74375) (width 0.381) (layer F.Cu) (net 9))
 (via (at 146.558 110.49) (size 0.8) (drill 0.4) (layers F.Cu B.Cu) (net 9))
 (segment (start 146.573 110.475) (end 146.558 110.49) (width 0.381) (layer F.Cu) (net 9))
 (segment (start 146.573 107.823) (end 146.573 110.475) (width 0.381) (layer F.Cu) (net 9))
 (segment (start 146.558 110.49) (end 150.114 110.49) (width 0.381) (layer B.Cu) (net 9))
 (segment (start 150.114 110.49) (end 150.114 95.631) (width 0.381) (layer B.Cu) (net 9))
 (segment (start 150.114 95.631) (end 141.859 95.631) (width 0.381) (layer B.Cu) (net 9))
 (segment (start 141.859 95.631) (end 141.859 97.155) (width 0.381) (layer B.Cu) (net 9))
 (segment (start 128.784 90.926) (end 131.445 90.926) (width 0.381) (layer F.Cu) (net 5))
 (segment (start 124.333 95.377) (end 128.784 90.926) (width 0.381) (layer F.Cu) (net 5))
 (segment (start 118.02725 93.699596) (end 119.704654 95.377) (width 0.381) (layer F.Cu) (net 5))
 (segment (start 119.704654 95.377) (end 124.333 95.377) (width 0.381) (layer F.Cu) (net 5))
 (segment (start 118.02725 93.49525) (end 118.02725 93.699596) (width 0.381) (layer F.Cu) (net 5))
 (segment (start 126.821 115.5515) (end 126.746 115.4765) (width 0.254) (layer F.Cu) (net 9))
 (segment (start 126.746 115.4765) (end 135.2215 115.4765) (width 0.381) (layer F.Cu) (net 9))
 (segment (start 135.4585 115.2395) (end 135.4585 108.98275) (width 0.381) (layer F.Cu) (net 9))
 (segment (start 135.2215 115.4765) (end 135.4585 115.2395) (width 0.381) (layer F.Cu) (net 9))
 (segment (start 145.23275 106.48275) (end 143.5585 106.48275) (width 0.381) (layer F.Cu) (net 9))
 (segment (start 146.573 107.823) (end 145.23275 106.48275) (width 0.381) (layer F.Cu) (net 9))
 (segment (start 131.017999 98.558251) (end 132.598 96.97825) (width 0.381) (layer F.Cu) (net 9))
 (segment (start 131.017999 100.073249) (end 131.017999 98.558251) (width 0.381) (layer F.Cu) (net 9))
 (segment (start 131.0275 100.08275) (end 131.017999 100.073249) (width 0.381) (layer F.Cu) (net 9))
 (segment (start 132.1585 100.08275) (end 131.0275 100.08275) (width 0.381) (layer F.Cu) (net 9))
 (segment (start 133.8585 98.71375) (end 133.8585 97.58275) (width 0.381) (layer F.Cu) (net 9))
 (segment (start 133.8585 99.51375) (end 133.8585 98.71375) (width 0.381) (layer F.Cu) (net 9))
 (segment (start 133.2895 100.08275) (end 133.8585 99.51375) (width 0.381) (layer F.Cu) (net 9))
 (segment (start 132.1585 100.08275) (end 133.2895 100.08275) (width 0.381) (layer F.Cu) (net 9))
 (segment (start 135.4585 107.85175) (end 135.4585 108.98275) (width 0.381) (layer F.Cu) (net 9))
 (segment (start 135.4585 106.25175) (end 135.4585 107.85175) (width 0.381) (layer F.Cu) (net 9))
 (segment (start 133.2895 104.08275) (end 135.4585 106.25175) (width 0.381) (layer F.Cu) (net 9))
 (segment (start 132.1585 104.08275) (end 133.2895 104.08275) (width 0.381) (layer F.Cu) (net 9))
 (segment (start 125.667 120.48275) (end 124.43725 119.253) (width 0.254) (layer F.Cu) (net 31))
 (segment (start 126.821 120.48275) (end 125.667 120.48275) (width 0.254) (layer F.Cu) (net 31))
 (segment (start 124.43725 115.91025) (end 124.46 115.8875) (width 0.254) (layer F.Cu) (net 31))
 (segment (start 124.43725 119.253) (end 124.43725 115.91025) (width 0.254) (layer F.Cu) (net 31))
 (segment (start 124.46 115.8875) (end 124.46 113.792) (width 0.254) (layer F.Cu) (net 31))
 (segment (start 124.6505 113.6015) (end 126.746 113.6015) (width 0.254) (layer F.Cu) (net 31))
 (segment (start 124.46 113.792) (end 124.6505 113.6015) (width 0.254) (layer F.Cu) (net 31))
 (segment (start 134.6585 109.98675) (end 134.6585 108.98275) (width 0.254) (layer F.Cu) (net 31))
 (segment (start 131.04375 113.6015) (end 134.6585 109.98675) (width 0.254) (layer F.Cu) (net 31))
 (segment (start 126.746 113.6015) (end 131.04375 113.6015) (width 0.254) (layer F.Cu) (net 31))
 (segment (start 116.42725 95.66275) (end 115.443 96.647) (width 0.254) (layer F.Cu) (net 7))
 (segment (start 116.42725 93.49525) (end 116.42725 95.66275) (width 0.254) (layer F.Cu) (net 7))
 (segment (start 115.443 98.522) (end 115.443 99.0095) (width 0.254) (layer F.Cu) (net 38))
 (segment (start 118.11625 101.68275) (end 132.1585 101.68275) (width 0.254) (layer F.Cu) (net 38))
 (segment (start 115.443 99.0095) (end 118.11625 101.68275) (width 0.254) (layer F.Cu) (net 38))
 (segment (start 117.22725 95.5085) (end 118.26875 96.55) (width 0.254) (layer F.Cu) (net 6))
 (segment (start 117.22725 93.49525) (end 117.22725 95.5085) (width 0.254) (layer F.Cu) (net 6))
 (segment (start 131.1545 100.88275) (end 132.1585 100.88275) (width 0.254) (layer F.Cu) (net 39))
 (segment (start 120.239 100.88275) (end 131.1545 100.88275) (width 0.254) (layer F.Cu) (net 39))
 (segment (start 118.26875 98.9125) (end 120.239 100.88275) (width 0.254) (layer F.Cu) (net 39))
 (segment (start 118.26875 98.425) (end 118.26875 98.9125) (width 0.254) (layer F.Cu) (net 39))
 (segment (start 143.5585 98.75375) (end 143.5585 99.28275) (width 0.254) (layer F.Cu) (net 17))
 (segment (start 143.792 98.52025) (end 143.5585 98.75375) (width 0.254) (layer F.Cu) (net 17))
 (segment (start 146.7485 98.52025) (end 143.792 98.52025) (width 0.254) (layer F.Cu) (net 17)))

